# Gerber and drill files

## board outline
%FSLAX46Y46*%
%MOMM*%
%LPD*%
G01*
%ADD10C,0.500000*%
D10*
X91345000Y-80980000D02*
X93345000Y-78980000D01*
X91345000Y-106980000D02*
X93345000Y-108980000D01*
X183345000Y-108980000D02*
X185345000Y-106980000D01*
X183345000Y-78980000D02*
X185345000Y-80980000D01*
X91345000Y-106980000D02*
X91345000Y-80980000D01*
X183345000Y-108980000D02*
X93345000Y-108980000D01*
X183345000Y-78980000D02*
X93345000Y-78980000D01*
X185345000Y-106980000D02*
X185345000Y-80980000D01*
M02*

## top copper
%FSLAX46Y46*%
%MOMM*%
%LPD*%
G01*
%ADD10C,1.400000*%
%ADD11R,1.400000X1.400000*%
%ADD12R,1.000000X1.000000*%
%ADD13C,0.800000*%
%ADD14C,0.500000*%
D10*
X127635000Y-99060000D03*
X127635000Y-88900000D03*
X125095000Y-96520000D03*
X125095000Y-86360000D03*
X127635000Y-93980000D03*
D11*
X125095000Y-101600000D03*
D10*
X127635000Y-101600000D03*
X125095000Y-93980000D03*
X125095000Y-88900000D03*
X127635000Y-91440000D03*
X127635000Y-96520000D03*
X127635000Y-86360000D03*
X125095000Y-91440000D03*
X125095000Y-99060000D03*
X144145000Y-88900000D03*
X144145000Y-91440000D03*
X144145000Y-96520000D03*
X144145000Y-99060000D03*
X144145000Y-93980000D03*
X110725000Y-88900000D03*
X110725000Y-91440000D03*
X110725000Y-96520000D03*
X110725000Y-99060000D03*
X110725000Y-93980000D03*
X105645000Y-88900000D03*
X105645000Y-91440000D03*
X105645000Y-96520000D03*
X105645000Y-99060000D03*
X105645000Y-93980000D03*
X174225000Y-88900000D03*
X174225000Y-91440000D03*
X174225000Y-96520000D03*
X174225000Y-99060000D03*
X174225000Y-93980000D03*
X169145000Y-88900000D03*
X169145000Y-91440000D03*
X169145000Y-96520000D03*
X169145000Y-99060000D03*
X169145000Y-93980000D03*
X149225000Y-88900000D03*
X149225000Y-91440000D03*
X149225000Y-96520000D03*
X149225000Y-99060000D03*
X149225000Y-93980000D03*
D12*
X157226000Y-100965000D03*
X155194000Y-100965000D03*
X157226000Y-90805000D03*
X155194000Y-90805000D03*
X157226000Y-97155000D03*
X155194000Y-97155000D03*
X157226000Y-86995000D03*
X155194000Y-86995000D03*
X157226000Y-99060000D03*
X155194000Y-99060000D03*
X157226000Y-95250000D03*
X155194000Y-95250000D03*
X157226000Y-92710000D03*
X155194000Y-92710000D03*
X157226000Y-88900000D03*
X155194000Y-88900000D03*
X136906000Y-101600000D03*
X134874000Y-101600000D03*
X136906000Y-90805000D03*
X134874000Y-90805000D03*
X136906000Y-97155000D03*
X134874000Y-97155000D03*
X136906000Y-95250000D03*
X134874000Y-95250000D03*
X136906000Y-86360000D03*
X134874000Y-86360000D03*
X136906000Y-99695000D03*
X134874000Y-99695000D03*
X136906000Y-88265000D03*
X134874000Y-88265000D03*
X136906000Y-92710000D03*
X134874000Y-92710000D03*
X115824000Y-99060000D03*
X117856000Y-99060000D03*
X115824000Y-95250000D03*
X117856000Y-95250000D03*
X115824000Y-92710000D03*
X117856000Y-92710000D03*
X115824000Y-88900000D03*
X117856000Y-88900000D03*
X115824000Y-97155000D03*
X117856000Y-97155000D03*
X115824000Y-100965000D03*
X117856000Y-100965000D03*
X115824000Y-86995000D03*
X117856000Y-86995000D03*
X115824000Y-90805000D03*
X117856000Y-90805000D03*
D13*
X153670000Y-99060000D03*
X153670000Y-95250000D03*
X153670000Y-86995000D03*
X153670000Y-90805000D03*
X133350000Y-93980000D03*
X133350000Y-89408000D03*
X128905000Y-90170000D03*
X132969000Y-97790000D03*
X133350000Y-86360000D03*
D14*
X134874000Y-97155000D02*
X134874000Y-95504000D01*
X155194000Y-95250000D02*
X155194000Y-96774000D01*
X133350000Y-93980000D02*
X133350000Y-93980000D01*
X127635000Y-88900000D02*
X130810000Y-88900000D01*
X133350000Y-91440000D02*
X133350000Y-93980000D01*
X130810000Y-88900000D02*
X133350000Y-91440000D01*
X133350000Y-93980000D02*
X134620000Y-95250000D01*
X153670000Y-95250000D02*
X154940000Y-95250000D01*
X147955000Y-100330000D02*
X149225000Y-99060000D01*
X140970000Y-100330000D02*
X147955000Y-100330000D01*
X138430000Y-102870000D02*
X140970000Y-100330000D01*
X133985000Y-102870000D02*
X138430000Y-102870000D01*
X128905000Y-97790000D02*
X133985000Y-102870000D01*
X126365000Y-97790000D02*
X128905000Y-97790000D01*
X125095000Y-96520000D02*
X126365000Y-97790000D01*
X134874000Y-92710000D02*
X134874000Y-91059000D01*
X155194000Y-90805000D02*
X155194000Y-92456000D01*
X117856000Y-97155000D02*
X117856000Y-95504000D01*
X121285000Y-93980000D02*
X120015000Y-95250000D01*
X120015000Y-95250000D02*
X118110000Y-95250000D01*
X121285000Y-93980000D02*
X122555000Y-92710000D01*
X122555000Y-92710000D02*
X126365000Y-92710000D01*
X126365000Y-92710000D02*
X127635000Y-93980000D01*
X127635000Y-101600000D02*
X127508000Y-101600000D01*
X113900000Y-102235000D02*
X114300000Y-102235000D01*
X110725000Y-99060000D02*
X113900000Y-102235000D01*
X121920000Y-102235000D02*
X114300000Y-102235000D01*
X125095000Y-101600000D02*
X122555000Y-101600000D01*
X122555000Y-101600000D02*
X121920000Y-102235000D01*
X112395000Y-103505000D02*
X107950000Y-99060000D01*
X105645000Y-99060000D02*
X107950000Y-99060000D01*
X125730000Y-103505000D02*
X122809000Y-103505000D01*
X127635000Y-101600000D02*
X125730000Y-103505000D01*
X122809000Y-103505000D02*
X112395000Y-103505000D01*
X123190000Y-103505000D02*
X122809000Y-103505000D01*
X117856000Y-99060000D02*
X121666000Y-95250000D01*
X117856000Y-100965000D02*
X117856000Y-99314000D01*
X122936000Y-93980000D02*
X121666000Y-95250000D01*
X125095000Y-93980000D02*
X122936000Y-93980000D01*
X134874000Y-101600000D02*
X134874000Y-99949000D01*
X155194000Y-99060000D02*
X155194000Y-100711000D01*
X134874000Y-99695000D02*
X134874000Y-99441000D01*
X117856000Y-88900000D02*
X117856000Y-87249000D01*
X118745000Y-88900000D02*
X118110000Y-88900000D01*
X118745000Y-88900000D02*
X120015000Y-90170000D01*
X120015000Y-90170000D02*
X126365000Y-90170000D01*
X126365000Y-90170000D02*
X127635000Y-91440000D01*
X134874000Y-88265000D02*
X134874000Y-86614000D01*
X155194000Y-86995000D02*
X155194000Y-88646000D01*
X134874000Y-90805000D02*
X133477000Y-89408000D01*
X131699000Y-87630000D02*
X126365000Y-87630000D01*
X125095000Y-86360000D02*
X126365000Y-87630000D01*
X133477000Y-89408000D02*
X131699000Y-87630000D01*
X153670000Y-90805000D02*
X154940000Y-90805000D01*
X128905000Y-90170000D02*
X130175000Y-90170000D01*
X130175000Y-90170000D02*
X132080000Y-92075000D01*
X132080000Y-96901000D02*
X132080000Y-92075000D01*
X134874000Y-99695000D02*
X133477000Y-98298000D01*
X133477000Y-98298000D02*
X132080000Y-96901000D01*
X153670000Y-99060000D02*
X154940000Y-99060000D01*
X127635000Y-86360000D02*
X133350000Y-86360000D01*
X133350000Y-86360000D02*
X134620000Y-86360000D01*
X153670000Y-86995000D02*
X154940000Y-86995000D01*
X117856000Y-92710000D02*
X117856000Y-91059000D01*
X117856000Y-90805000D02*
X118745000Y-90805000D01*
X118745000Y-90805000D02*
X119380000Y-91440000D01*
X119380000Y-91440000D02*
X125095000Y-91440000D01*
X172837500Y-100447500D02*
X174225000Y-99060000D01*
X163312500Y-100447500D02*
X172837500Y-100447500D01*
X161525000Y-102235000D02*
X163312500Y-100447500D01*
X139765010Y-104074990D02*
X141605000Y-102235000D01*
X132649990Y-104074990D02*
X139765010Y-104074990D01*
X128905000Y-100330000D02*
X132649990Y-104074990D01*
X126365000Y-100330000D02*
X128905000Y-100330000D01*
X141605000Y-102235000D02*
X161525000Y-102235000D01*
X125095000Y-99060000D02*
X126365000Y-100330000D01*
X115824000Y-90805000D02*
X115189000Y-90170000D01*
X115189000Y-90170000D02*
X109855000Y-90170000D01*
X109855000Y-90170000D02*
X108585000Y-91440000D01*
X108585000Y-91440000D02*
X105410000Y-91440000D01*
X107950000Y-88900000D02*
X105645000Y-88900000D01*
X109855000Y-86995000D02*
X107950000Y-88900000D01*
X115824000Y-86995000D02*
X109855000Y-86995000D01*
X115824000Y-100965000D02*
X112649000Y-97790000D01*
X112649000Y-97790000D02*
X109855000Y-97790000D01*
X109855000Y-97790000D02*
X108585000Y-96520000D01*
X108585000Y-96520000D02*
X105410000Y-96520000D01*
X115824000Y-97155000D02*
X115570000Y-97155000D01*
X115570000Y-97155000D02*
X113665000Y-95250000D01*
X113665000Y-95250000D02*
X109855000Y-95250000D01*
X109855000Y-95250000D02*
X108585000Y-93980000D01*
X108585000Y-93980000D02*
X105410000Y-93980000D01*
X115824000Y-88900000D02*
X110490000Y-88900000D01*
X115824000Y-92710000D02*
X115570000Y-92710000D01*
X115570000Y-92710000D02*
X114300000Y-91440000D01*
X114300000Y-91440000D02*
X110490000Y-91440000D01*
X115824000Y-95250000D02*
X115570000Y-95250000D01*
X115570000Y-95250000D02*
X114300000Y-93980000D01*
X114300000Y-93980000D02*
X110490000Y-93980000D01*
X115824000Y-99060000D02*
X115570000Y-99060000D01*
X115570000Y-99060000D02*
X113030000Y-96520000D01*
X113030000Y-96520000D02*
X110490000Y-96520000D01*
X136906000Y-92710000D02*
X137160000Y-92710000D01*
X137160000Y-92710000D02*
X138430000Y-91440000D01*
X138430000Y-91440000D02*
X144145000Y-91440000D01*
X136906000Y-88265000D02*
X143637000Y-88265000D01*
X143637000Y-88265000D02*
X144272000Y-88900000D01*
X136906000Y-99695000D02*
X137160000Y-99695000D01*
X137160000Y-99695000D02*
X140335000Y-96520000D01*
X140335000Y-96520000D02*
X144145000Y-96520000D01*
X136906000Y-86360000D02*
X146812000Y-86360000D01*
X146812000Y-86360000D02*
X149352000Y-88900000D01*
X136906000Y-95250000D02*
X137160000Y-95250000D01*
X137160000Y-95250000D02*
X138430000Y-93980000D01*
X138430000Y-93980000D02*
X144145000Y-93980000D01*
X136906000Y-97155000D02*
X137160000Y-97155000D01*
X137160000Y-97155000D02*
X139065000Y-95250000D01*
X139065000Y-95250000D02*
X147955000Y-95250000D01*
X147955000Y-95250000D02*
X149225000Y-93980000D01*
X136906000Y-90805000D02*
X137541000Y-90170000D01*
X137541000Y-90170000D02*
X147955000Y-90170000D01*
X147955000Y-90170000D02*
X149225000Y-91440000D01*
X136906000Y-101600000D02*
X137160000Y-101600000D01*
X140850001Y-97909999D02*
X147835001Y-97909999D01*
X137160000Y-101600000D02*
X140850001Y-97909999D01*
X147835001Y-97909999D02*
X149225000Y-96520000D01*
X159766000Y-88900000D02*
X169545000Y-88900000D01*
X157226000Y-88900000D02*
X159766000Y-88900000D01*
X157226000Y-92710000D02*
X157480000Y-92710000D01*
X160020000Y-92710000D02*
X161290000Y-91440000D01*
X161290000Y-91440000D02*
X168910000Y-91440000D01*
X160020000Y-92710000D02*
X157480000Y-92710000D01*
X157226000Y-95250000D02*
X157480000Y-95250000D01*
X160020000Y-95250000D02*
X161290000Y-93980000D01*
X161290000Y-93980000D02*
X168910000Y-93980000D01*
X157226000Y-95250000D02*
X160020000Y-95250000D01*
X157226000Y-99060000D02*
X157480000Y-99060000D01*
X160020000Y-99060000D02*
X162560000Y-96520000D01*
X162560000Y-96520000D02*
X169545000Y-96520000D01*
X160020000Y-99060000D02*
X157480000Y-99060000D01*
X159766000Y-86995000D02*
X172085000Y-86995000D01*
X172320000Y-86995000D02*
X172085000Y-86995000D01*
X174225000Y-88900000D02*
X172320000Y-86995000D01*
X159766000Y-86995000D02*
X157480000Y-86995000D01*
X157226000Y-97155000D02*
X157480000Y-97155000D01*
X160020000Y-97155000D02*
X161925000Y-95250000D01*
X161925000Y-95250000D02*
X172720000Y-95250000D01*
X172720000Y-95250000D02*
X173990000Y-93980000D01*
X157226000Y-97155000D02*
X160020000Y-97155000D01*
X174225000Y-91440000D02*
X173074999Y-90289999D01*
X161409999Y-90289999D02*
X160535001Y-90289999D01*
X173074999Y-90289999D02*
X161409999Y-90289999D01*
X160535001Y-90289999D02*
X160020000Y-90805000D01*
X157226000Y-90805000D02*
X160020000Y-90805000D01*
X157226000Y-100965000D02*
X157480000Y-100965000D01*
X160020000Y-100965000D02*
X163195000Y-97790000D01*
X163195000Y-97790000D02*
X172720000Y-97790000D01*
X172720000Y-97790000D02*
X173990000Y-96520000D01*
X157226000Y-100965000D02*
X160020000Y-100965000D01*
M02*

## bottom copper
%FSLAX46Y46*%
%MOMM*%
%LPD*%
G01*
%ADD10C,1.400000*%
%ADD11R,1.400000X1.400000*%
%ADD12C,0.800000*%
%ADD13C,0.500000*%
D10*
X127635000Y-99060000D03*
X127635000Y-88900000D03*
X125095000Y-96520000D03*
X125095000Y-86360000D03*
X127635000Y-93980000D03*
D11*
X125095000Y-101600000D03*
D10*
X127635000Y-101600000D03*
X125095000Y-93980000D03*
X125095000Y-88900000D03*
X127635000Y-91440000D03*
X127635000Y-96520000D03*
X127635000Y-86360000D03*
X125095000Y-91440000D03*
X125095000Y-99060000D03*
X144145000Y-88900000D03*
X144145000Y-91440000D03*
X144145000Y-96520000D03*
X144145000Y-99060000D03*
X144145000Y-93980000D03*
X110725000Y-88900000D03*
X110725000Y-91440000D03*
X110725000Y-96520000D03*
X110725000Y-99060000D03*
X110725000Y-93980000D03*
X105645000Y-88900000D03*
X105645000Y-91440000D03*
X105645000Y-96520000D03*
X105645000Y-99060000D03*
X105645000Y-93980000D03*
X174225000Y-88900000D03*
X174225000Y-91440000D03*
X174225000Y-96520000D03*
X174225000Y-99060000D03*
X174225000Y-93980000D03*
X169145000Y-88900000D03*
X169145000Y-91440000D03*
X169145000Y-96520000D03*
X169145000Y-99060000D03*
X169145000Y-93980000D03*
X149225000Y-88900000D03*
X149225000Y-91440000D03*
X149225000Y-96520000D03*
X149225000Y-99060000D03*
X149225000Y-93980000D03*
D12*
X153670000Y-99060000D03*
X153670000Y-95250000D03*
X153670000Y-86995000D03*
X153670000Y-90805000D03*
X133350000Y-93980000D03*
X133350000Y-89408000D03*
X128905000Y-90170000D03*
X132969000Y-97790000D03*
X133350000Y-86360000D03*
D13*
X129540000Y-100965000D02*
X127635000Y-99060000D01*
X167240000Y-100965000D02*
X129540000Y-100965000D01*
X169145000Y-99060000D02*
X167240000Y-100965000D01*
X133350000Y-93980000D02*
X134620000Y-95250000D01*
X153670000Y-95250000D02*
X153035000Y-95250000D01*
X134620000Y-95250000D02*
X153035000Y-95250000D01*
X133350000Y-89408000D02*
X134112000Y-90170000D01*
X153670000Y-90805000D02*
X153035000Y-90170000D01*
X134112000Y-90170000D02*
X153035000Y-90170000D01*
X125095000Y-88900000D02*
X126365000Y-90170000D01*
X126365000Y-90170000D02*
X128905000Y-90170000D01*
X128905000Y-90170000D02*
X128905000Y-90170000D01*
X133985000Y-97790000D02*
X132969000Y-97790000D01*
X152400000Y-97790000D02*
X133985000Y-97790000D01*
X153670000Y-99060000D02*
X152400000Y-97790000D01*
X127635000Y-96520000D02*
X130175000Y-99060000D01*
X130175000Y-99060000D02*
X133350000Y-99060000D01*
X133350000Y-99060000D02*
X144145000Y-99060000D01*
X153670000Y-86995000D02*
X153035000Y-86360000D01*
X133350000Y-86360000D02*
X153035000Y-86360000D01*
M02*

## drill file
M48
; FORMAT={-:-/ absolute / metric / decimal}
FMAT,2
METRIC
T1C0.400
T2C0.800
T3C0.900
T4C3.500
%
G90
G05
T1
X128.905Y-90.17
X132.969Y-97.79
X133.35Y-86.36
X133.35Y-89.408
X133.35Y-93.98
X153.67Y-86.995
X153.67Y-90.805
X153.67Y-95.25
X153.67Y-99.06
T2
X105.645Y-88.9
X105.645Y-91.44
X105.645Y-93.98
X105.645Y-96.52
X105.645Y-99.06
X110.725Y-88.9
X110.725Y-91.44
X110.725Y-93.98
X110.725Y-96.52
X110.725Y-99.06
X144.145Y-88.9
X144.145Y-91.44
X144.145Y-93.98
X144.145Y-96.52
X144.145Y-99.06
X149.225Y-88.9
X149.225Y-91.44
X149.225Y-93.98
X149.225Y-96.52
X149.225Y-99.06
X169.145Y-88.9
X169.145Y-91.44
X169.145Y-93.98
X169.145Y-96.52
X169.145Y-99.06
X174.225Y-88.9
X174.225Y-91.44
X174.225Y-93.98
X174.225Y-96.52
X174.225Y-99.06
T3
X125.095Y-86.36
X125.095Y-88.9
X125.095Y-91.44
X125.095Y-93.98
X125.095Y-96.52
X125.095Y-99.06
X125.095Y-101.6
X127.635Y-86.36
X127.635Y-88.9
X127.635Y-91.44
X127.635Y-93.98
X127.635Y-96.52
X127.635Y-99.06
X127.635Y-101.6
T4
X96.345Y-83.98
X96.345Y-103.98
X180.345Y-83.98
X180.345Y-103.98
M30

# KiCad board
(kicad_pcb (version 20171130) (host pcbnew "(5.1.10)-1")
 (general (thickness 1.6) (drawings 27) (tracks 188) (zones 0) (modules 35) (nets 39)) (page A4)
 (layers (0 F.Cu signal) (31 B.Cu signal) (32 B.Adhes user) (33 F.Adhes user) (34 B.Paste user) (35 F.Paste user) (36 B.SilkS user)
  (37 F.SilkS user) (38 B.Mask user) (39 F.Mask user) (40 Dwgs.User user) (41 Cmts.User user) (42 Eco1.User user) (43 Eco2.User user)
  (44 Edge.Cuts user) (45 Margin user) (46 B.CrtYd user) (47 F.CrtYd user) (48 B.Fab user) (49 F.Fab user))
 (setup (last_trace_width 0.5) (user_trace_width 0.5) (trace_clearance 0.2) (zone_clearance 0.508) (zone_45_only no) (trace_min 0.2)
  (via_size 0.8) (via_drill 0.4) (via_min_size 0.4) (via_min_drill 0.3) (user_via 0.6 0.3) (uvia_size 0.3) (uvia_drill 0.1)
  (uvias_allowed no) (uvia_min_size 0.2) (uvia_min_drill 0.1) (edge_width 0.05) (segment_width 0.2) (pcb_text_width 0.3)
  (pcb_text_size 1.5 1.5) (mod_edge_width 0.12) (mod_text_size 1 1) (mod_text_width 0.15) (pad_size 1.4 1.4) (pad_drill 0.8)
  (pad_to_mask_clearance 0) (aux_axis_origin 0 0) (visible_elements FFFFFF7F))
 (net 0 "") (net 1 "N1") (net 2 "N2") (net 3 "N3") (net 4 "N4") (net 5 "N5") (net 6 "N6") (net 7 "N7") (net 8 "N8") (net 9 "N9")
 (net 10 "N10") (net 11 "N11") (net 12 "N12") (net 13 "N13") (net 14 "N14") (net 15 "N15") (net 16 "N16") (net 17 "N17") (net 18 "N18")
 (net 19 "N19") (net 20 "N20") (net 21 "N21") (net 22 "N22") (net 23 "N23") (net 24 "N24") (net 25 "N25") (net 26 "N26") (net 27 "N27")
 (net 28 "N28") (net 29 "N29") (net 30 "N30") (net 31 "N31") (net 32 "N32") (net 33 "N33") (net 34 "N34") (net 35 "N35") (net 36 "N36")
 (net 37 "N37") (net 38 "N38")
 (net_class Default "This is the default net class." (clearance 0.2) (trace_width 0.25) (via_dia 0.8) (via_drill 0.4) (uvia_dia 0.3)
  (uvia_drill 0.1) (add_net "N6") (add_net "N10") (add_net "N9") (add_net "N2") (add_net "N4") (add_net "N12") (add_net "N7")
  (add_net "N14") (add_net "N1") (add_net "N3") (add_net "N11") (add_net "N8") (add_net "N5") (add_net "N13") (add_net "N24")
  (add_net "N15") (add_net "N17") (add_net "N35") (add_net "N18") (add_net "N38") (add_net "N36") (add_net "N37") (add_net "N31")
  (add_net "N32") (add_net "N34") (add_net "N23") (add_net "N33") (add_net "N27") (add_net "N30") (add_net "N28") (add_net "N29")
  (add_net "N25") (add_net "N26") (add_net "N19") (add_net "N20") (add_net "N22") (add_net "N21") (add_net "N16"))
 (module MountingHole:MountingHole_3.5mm (layer F.Cu) (at 96.345 103.98)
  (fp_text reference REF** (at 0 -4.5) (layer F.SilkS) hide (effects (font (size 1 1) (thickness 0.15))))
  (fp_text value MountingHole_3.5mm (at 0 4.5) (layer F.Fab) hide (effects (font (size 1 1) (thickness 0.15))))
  (pad 1 np_thru_hole circle (at 0 0) (size 3.5 3.5) (drill 3.5) (layers *.Cu *.Mask)))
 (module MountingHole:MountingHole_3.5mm (layer F.Cu) (at 96.345 83.98)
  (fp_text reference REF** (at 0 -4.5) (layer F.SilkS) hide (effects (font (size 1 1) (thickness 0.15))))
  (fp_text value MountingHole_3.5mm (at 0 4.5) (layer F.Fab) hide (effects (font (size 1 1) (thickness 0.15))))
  (pad 1 np_thru_hole circle (at 0 0) (size 3.5 3.5) (drill 3.5) (layers *.Cu *.Mask)))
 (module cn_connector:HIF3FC (layer B.Cu) (at 126.365 93.98)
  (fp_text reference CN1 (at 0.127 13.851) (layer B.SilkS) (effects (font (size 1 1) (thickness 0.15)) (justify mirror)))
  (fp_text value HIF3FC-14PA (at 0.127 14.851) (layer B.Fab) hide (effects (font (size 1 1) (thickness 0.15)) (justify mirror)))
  (pad 4 thru_hole circle (at 1.27 5.08) (size 1.4 1.4) (drill 0.9) (layers *.Cu *.Mask) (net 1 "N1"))
  (pad 12 thru_hole circle (at 1.27 -5.08) (size 1.4 1.4) (drill 0.9) (layers *.Cu *.Mask) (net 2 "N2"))
  (pad 5 thru_hole circle (at -1.27 2.54) (size 1.4 1.4) (drill 0.9) (layers *.Cu *.Mask) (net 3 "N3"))
  (pad 13 thru_hole circle (at -1.27 -7.62) (size 1.4 1.4) (drill 0.9) (layers *.Cu *.Mask) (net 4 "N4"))
  (pad 8 thru_hole circle (at 1.27 0) (size 1.4 1.4) (drill 0.9) (layers *.Cu *.Mask) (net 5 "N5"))
  (pad 1 thru_hole rect (at -1.27 7.62) (size 1.4 1.4) (drill 0.9) (layers *.Cu *.Mask) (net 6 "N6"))
  (pad 2 thru_hole circle (at 1.27 7.62) (size 1.4 1.4) (drill 0.9) (layers *.Cu *.Mask) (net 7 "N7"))
  (pad 7 thru_hole circle (at -1.27 0) (size 1.4 1.4) (drill 0.9) (layers *.Cu *.Mask) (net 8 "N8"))
  (pad 11 thru_hole circle (at -1.27 -5.08) (size 1.4 1.4) (drill 0.9) (layers *.Cu *.Mask) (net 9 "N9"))
  (pad 10 thru_hole circle (at 1.27 -2.54) (size 1.4 1.4) (drill 0.9) (layers *.Cu *.Mask) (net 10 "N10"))
  (pad 6 thru_hole circle (at 1.27 2.54) (size 1.4 1.4) (drill 0.9) (layers *.Cu *.Mask) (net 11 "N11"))
  (pad 14 thru_hole circle (at 1.27 -7.62) (size 1.4 1.4) (drill 0.9) (layers *.Cu *.Mask) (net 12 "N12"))
  (pad 9 thru_hole circle (at -1.27 -2.54) (size 1.4 1.4) (drill 0.9) (layers *.Cu *.Mask) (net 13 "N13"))
  (pad 3 thru_hole circle (at -1.27 5.08) (size 1.4 1.4) (drill 0.9) (layers *.Cu *.Mask) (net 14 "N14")))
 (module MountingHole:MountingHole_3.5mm (layer F.Cu) (at 180.345 103.98)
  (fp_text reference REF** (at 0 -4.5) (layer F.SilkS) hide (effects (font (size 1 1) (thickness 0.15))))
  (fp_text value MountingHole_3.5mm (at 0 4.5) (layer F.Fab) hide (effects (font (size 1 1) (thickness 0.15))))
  (pad 1 np_thru_hole circle (at 0 0) (size 3.5 3.5) (drill 3.5) (layers *.Cu *.Mask)))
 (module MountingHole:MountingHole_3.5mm (layer F.Cu) (at 180.345 83.98)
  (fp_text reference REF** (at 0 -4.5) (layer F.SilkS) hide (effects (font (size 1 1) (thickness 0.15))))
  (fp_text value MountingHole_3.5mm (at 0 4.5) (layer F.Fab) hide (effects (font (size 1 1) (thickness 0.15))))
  (pad 1 np_thru_hole circle (at 0 0) (size 3.5 3.5) (drill 3.5) (layers *.Cu *.Mask)))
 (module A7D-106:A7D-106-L (layer F.Cu) (at 144.145 88.9)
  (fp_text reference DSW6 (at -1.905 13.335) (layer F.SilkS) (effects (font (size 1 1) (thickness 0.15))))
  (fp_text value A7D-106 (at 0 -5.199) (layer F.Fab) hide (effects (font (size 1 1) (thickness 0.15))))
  (pad 8 thru_hole circle (at 0 0) (size 1.4 1.4) (drill 0.8) (layers *.Cu *.Mask) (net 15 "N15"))
  (pad 4 thru_hole circle (at 0 2.54) (size 1.4 1.4) (drill 0.8) (layers *.Cu *.Mask) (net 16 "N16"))
  (pad 1 thru_hole circle (at 0 7.62) (size 1.4 1.4) (drill 0.8) (layers *.Cu *.Mask) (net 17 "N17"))
  (pad C thru_hole circle (at 0 10.16) (size 1.4 1.4) (drill 0.8) (layers *.Cu *.Mask) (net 11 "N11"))
  (pad 2 thru_hole circle (at 0 5.08) (size 1.4 1.4) (drill 0.8) (layers *.Cu *.Mask) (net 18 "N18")))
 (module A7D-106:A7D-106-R (layer F.Cu) (at 110.725 88.9)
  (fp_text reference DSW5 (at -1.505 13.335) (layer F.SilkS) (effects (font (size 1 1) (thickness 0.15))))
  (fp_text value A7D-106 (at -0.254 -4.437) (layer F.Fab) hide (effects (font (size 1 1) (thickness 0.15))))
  (pad 8 thru_hole circle (at 0 0) (size 1.4 1.4) (drill 0.8) (layers *.Cu *.Mask) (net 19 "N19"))
  (pad 4 thru_hole circle (at 0 2.54) (size 1.4 1.4) (drill 0.8) (layers *.Cu *.Mask) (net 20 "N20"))
  (pad 1 thru_hole circle (at 0 7.62) (size 1.4 1.4) (drill 0.8) (layers *.Cu *.Mask) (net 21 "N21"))
  (pad C thru_hole circle (at 0 10.16) (size 1.4 1.4) (drill 0.8) (layers *.Cu *.Mask) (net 6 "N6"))
  (pad 2 thru_hole circle (at 0 5.08) (size 1.4 1.4) (drill 0.8) (layers *.Cu *.Mask) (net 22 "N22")))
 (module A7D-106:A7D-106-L (layer F.Cu) (at 105.645 88.9)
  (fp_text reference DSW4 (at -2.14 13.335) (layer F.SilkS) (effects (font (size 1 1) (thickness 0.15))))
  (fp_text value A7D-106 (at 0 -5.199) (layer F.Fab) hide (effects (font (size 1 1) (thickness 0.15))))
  (pad 8 thru_hole circle (at 0 0) (size 1.4 1.4) (drill 0.8) (layers *.Cu *.Mask) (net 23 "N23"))
  (pad 4 thru_hole circle (at 0 2.54) (size 1.4 1.4) (drill 0.8) (layers *.Cu *.Mask) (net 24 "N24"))
  (pad 1 thru_hole circle (at 0 7.62) (size 1.4 1.4) (drill 0.8) (layers *.Cu *.Mask) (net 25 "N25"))
  (pad C thru_hole circle (at 0 10.16) (size 1.4 1.4) (drill 0.8) (layers *.Cu *.Mask) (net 7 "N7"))
  (pad 2 thru_hole circle (at 0 5.08) (size 1.4 1.4) (drill 0.8) (layers *.Cu *.Mask) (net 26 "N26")))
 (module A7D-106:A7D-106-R (layer F.Cu) (at 174.225 88.9)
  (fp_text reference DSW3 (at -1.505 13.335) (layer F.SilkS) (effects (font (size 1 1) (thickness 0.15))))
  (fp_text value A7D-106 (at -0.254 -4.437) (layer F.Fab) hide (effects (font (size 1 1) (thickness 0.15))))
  (pad 8 thru_hole circle (at 0 0) (size 1.4 1.4) (drill 0.8) (layers *.Cu *.Mask) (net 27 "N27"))
  (pad 4 thru_hole circle (at 0 2.54) (size 1.4 1.4) (drill 0.8) (layers *.Cu *.Mask) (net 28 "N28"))
  (pad 1 thru_hole circle (at 0 7.62) (size 1.4 1.4) (drill 0.8) (layers *.Cu *.Mask) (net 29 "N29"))
  (pad C thru_hole circle (at 0 10.16) (size 1.4 1.4) (drill 0.8) (layers *.Cu *.Mask) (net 14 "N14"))
  (pad 2 thru_hole circle (at 0 5.08) (size 1.4 1.4) (drill 0.8) (layers *.Cu *.Mask) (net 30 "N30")))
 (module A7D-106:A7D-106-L (layer F.Cu) (at 169.145 88.9)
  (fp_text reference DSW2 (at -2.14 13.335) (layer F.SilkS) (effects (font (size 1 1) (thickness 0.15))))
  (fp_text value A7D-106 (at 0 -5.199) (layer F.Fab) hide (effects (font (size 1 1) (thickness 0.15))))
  (pad 8 thru_hole circle (at 0 0) (size 1.4 1.4) (drill 0.8) (layers *.Cu *.Mask) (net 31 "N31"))
  (pad 4 thru_hole circle (at 0 2.54) (size 1.4 1.4) (drill 0.8) (layers *.Cu *.Mask) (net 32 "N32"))
  (pad 1 thru_hole circle (at 0 7.62) (size 1.4 1.4) (drill 0.8) (layers *.Cu *.Mask) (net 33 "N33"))
  (pad C thru_hole circle (at 0 10.16) (size 1.4 1.4) (drill 0.8) (layers *.Cu *.Mask) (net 1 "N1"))
  (pad 2 thru_hole circle (at 0 5.08) (size 1.4 1.4) (drill 0.8) (layers *.Cu *.Mask) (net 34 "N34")))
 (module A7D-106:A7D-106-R (layer F.Cu) (at 149.225 88.9)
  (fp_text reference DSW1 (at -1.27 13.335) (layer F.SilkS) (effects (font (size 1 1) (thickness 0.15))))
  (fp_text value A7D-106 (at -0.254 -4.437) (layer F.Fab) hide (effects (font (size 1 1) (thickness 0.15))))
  (pad 8 thru_hole circle (at 0 0) (size 1.4 1.4) (drill 0.8) (layers *.Cu *.Mask) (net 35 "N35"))
  (pad 4 thru_hole circle (at 0 2.54) (size 1.4 1.4) (drill 0.8) (layers *.Cu *.Mask) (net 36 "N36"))
  (pad 1 thru_hole circle (at 0 7.62) (size 1.4 1.4) (drill 0.8) (layers *.Cu *.Mask) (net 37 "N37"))
  (pad C thru_hole circle (at 0 10.16) (size 1.4 1.4) (drill 0.8) (layers *.Cu *.Mask) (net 3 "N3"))
  (pad 2 thru_hole circle (at 0 5.08) (size 1.4 1.4) (drill 0.8) (layers *.Cu *.Mask) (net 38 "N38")))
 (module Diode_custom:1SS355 (layer F.Cu) (at 156.21 100.965)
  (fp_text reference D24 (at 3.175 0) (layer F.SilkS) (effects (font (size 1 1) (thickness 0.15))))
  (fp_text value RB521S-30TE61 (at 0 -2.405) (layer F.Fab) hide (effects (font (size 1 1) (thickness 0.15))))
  (pad 2 smd rect (at 1.016 0) (size 1 1) (layers F.Cu F.Paste F.Mask) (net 29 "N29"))
  (pad 1 smd rect (at -1.016 0) (size 1 1) (layers F.Cu F.Paste F.Mask) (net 9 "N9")))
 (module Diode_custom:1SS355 (layer F.Cu) (at 156.21 90.805)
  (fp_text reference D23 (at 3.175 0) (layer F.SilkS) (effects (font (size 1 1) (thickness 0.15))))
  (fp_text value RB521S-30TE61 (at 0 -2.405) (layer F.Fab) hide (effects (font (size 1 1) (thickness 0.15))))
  (pad 2 smd rect (at 1.016 0) (size 1 1) (layers F.Cu F.Paste F.Mask) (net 28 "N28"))
  (pad 1 smd rect (at -1.016 0) (size 1 1) (layers F.Cu F.Paste F.Mask) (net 4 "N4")))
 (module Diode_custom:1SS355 (layer F.Cu) (at 156.21 97.155)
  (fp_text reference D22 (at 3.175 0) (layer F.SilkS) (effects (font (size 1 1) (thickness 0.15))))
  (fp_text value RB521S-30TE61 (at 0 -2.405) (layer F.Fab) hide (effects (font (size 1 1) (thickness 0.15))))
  (pad 2 smd rect (at 1.016 0) (size 1 1) (layers F.Cu F.Paste F.Mask) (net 30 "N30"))
  (pad 1 smd rect (at -1.016 0) (size 1 1) (layers F.Cu F.Paste F.Mask) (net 2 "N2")))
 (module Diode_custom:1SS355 (layer F.Cu) (at 156.21 86.995)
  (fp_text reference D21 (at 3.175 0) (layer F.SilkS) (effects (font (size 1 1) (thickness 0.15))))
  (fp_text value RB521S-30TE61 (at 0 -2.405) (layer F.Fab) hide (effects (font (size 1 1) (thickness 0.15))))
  (pad 2 smd rect (at 1.016 0) (size 1 1) (layers F.Cu F.Paste F.Mask) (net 27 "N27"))
  (pad 1 smd rect (at -1.016 0) (size 1 1) (layers F.Cu F.Paste F.Mask) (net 12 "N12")))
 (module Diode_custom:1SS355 (layer F.Cu) (at 156.21 99.06)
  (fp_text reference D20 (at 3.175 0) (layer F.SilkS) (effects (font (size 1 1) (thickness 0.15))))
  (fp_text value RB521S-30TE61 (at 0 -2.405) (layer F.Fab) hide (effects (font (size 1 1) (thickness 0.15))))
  (pad 2 smd rect (at 1.016 0) (size 1 1) (layers F.Cu F.Paste F.Mask) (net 33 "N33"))
  (pad 1 smd rect (at -1.016 0) (size 1 1) (layers F.Cu F.Paste F.Mask) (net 9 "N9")))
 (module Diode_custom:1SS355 (layer F.Cu) (at 156.21 95.25)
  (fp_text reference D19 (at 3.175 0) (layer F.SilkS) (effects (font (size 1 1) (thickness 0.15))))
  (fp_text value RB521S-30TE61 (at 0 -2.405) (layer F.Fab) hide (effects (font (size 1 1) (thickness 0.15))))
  (pad 2 smd rect (at 1.016 0) (size 1 1) (layers F.Cu F.Paste F.Mask) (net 34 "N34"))
  (pad 1 smd rect (at -1.016 0) (size 1 1) (layers F.Cu F.Paste F.Mask) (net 2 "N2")))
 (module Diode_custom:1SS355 (layer F.Cu) (at 156.21 92.71)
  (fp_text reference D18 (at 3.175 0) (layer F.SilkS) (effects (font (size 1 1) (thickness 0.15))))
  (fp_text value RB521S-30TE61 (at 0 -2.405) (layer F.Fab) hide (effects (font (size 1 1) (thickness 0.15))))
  (pad 2 smd rect (at 1.016 0) (size 1 1) (layers F.Cu F.Paste F.Mask) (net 32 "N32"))
  (pad 1 smd rect (at -1.016 0) (size 1 1) (layers F.Cu F.Paste F.Mask) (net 4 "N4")))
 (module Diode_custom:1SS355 (layer F.Cu) (at 156.21 88.9)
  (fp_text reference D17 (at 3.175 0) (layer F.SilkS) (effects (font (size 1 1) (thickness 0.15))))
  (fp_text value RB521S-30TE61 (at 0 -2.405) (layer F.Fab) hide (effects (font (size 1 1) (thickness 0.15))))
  (pad 2 smd rect (at 1.016 0) (size 1 1) (layers F.Cu F.Paste F.Mask) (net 31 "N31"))
  (pad 1 smd rect (at -1.016 0) (size 1 1) (layers F.Cu F.Paste F.Mask) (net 12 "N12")))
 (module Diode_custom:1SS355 (layer F.Cu) (at 135.89 101.6)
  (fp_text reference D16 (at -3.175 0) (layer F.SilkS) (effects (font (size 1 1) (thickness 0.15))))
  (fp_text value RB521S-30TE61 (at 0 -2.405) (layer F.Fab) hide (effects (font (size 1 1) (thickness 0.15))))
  (pad 2 smd rect (at 1.016 0) (size 1 1) (layers F.Cu F.Paste F.Mask) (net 37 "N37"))
  (pad 1 smd rect (at -1.016 0) (size 1 1) (layers F.Cu F.Paste F.Mask) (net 9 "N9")))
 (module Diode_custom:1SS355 (layer F.Cu) (at 135.89 90.805)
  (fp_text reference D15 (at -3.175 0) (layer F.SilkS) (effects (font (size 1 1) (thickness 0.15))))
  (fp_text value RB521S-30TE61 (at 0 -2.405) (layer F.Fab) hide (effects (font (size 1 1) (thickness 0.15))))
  (pad 2 smd rect (at 1.016 0) (size 1 1) (layers F.Cu F.Paste F.Mask) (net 36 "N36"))
  (pad 1 smd rect (at -1.016 0) (size 1 1) (layers F.Cu F.Paste F.Mask) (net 4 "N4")))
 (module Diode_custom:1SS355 (layer F.Cu) (at 135.89 97.155)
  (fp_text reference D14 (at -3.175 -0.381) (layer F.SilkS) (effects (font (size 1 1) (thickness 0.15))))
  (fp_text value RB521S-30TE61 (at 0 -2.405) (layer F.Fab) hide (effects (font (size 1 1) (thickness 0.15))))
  (pad 2 smd rect (at 1.016 0) (size 1 1) (layers F.Cu F.Paste F.Mask) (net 38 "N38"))
  (pad 1 smd rect (at -1.016 0) (size 1 1) (layers F.Cu F.Paste F.Mask) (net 2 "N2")))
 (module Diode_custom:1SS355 (layer F.Cu) (at 135.89 95.25)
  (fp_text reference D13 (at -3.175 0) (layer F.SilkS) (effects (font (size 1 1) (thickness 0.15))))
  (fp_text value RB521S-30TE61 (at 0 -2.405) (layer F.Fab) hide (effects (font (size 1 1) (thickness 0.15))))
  (pad 2 smd rect (at 1.016 0) (size 1 1) (layers F.Cu F.Paste F.Mask) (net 18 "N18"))
  (pad 1 smd rect (at -1.016 0) (size 1 1) (layers F.Cu F.Paste F.Mask) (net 2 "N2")))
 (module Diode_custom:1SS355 (layer F.Cu) (at 135.89 86.36)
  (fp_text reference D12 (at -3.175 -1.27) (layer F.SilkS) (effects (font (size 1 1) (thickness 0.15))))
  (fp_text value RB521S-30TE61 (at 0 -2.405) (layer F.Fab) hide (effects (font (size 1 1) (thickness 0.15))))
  (pad 2 smd rect (at 1.016 0) (size 1 1) (layers F.Cu F.Paste F.Mask) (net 35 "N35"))
  (pad 1 smd rect (at -1.016 0) (size 1 1) (layers F.Cu F.Paste F.Mask) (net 12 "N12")))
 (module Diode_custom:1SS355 (layer F.Cu) (at 135.89 99.695)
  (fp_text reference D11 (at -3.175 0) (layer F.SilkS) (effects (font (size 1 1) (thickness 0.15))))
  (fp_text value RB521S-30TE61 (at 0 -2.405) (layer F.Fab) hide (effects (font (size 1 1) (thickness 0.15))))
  (pad 2 smd rect (at 1.016 0) (size 1 1) (layers F.Cu F.Paste F.Mask) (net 17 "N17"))
  (pad 1 smd rect (at -1.016 0) (size 1 1) (layers F.Cu F.Paste F.Mask) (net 9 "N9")))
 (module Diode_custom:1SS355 (layer F.Cu) (at 135.89 88.265)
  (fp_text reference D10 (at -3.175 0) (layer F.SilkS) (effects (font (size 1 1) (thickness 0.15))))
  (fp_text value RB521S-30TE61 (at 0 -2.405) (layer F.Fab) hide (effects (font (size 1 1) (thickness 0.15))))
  (pad 2 smd rect (at 1.016 0) (size 1 1) (layers F.Cu F.Paste F.Mask) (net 15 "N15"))
  (pad 1 smd rect (at -1.016 0) (size 1 1) (layers F.Cu F.Paste F.Mask) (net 12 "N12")))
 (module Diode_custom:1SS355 (layer F.Cu) (at 135.89 92.71)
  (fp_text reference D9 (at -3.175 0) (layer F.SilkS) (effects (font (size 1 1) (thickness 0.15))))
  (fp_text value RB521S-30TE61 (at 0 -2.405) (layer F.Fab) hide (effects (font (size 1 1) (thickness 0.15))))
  (pad 2 smd rect (at 1.016 0) (size 1 1) (layers F.Cu F.Paste F.Mask) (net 16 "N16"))
  (pad 1 smd rect (at -1.016 0) (size 1 1) (layers F.Cu F.Paste F.Mask) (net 4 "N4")))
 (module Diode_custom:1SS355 (layer F.Cu) (at 116.84 99.06 180)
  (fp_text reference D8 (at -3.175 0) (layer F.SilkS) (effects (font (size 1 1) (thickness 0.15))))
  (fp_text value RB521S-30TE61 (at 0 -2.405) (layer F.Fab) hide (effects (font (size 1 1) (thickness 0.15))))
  (pad 2 smd rect (at 1.016 0 180) (size 1 1) (layers F.Cu F.Paste F.Mask) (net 21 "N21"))
  (pad 1 smd rect (at -1.016 0 180) (size 1 1) (layers F.Cu F.Paste F.Mask) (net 8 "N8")))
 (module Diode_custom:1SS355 (layer F.Cu) (at 116.84 95.25 180)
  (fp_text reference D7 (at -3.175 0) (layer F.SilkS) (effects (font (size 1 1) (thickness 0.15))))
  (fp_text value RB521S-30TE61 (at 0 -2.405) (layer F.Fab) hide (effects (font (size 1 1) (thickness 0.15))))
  (pad 2 smd rect (at 1.016 0 180) (size 1 1) (layers F.Cu F.Paste F.Mask) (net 22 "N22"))
  (pad 1 smd rect (at -1.016 0 180) (size 1 1) (layers F.Cu F.Paste F.Mask) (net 5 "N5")))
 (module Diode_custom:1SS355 (layer F.Cu) (at 116.84 92.71 180)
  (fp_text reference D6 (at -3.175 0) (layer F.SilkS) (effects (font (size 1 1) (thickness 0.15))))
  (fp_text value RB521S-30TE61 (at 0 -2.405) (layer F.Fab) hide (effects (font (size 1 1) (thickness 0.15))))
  (pad 2 smd rect (at 1.016 0 180) (size 1 1) (layers F.Cu F.Paste F.Mask) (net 20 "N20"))
  (pad 1 smd rect (at -1.016 0 180) (size 1 1) (layers F.Cu F.Paste F.Mask) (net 13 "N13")))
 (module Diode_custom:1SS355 (layer F.Cu) (at 116.84 88.9 180)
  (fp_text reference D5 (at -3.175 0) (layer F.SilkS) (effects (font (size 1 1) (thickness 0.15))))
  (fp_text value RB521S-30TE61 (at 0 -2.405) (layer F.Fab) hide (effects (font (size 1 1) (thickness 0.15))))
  (pad 2 smd rect (at 1.016 0 180) (size 1 1) (layers F.Cu F.Paste F.Mask) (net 19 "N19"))
  (pad 1 smd rect (at -1.016 0 180) (size 1 1) (layers F.Cu F.Paste F.Mask) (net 10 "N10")))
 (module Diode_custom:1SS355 (layer F.Cu) (at 116.84 97.155 180)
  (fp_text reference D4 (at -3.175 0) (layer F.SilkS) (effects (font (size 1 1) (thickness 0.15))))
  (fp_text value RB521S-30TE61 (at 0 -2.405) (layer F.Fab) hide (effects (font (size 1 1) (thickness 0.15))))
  (pad 2 smd rect (at 1.016 0 180) (size 1 1) (layers F.Cu F.Paste F.Mask) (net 26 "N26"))
  (pad 1 smd rect (at -1.016 0 180) (size 1 1) (layers F.Cu F.Paste F.Mask) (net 5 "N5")))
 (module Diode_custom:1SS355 (layer F.Cu) (at 116.84 100.965 180)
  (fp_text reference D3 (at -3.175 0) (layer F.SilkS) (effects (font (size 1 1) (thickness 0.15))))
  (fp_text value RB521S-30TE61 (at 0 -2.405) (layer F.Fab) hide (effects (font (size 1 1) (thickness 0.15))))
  (pad 2 smd rect (at 1.016 0 180) (size 1 1) (layers F.Cu F.Paste F.Mask) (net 25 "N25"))
  (pad 1 smd rect (at -1.016 0 180) (size 1 1) (layers F.Cu F.Paste F.Mask) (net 8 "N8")))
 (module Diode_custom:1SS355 (layer F.Cu) (at 116.84 86.995 180)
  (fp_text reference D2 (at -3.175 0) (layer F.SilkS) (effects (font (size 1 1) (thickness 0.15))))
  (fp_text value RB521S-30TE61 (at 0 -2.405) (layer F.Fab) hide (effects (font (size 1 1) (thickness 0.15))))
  (pad 2 smd rect (at 1.016 0 180) (size 1 1) (layers F.Cu F.Paste F.Mask) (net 23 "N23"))
  (pad 1 smd rect (at -1.016 0 180) (size 1 1) (layers F.Cu F.Paste F.Mask) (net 10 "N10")))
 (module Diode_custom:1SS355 (layer F.Cu) (at 116.84 90.805 180)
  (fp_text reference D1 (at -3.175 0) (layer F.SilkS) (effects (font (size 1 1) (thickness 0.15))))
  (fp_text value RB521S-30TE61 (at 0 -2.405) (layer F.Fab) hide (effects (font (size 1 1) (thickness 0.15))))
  (pad 2 smd rect (at 1.016 0 180) (size 1 1) (layers F.Cu F.Paste F.Mask) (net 24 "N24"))
  (pad 1 smd rect (at -1.016 0 180) (size 1 1) (layers F.Cu F.Paste F.Mask) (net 13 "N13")))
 (gr_line (start 91.345 80.98) (end 93.345 78.98) (layer Edge.Cuts) (width 0.5))
 (gr_line (start 91.345 106.98) (end 93.345 108.98) (layer Edge.Cuts) (width 0.5))
 (gr_line (start 183.345 108.98) (end 185.345 106.98) (layer Edge.Cuts) (width 0.5))
 (gr_line (start 183.345 78.98) (end 185.345 80.98) (layer Edge.Cuts) (width 0.5))
 (gr_line (start 91.345 106.98) (end 91.345 80.98) (layer Edge.Cuts) (width 0.5))
 (gr_line (start 183.345 108.98) (end 93.345 108.98) (layer Edge.Cuts) (width 0.5))
 (gr_line (start 183.345 78.98) (end 93.345 78.98) (layer Edge.Cuts) (width 0.5))
 (gr_line (start 185.345 106.98) (end 185.345 80.98) (layer Edge.Cuts) (width 0.5))
 (segment (start 129.54 100.965) (end 127.635 99.06) (width 0.5) (layer B.Cu) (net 1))
 (segment (start 167.24 100.965) (end 129.54 100.965) (width 0.5) (layer B.Cu) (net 1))
 (segment (start 169.145 99.06) (end 167.24 100.965) (width 0.5) (layer B.Cu) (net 1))
 (via (at 153.67 99.06) (size 0.8) (drill 0.4) (layers F.Cu B.Cu) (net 9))
 (via (at 153.67 95.25) (size 0.8) (drill 0.4) (layers F.Cu B.Cu) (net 2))
 (via (at 153.67 86.995) (size 0.8) (drill 0.4) (layers F.Cu B.Cu) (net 12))
 (via (at 153.67 90.805) (size 0.8) (drill 0.4) (layers F.Cu B.Cu) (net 4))
 (segment (start 134.874 97.155) (end 134.874 95.504) (width 0.5) (layer F.Cu) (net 2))
 (segment (start 155.194 95.25) (end 155.194 96.774) (width 0.5) (layer F.Cu) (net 2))
 (segment (start 133.35 93.98) (end 133.35 93.98) (width 0.5) (layer F.Cu) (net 2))
 (segment (start 127.635 88.9) (end 130.81 88.9) (width 0.5) (layer F.Cu) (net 2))
 (segment (start 133.35 91.44) (end 133.35 93.98) (width 0.5) (layer F.Cu) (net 2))
 (segment (start 130.81 88.9) (end 133.35 91.44) (width 0.5) (layer F.Cu) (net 2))
 (segment (start 133.35 93.98) (end 134.62 95.25) (width 0.5) (layer F.Cu) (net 2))
 (via (at 133.35 93.98) (size 0.8) (drill 0.4) (layers F.Cu B.Cu) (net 2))
 (segment (start 133.35 93.98) (end 134.62 95.25) (width 0.5) (layer B.Cu) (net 2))
 (segment (start 153.67 95.25) (end 153.035 95.25) (width 0.5) (layer B.Cu) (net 2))
 (segment (start 134.62 95.25) (end 153.035 95.25) (width 0.5) (layer B.Cu) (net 2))
 (segment (start 153.67 95.25) (end 154.94 95.25) (width 0.5) (layer F.Cu) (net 2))
 (segment (start 147.955 100.33) (end 149.225 99.06) (width 0.5) (layer F.Cu) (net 3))
 (segment (start 140.97 100.33) (end 147.955 100.33) (width 0.5) (layer F.Cu) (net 3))
 (segment (start 138.43 102.87) (end 140.97 100.33) (width 0.5) (layer F.Cu) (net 3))
 (segment (start 133.985 102.87) (end 138.43 102.87) (width 0.5) (layer F.Cu) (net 3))
 (segment (start 128.905 97.79) (end 133.985 102.87) (width 0.5) (layer F.Cu) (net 3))
 (segment (start 126.365 97.79) (end 128.905 97.79) (width 0.5) (layer F.Cu) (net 3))
 (segment (start 125.095 96.52) (end 126.365 97.79) (width 0.5) (layer F.Cu) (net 3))
 (segment (start 134.874 92.71) (end 134.874 91.059) (width 0.5) (layer F.Cu) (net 4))
 (segment (start 155.194 90.805) (end 155.194 92.456) (width 0.5) (layer F.Cu) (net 4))
 (segment (start 117.856 97.155) (end 117.856 95.504) (width 0.5) (layer F.Cu) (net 5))
 (segment (start 121.285 93.98) (end 120.015 95.25) (width 0.5) (layer F.Cu) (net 5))
 (segment (start 120.015 95.25) (end 118.11 95.25) (width 0.5) (layer F.Cu) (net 5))
 (segment (start 121.285 93.98) (end 122.555 92.71) (width 0.5) (layer F.Cu) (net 5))
 (segment (start 122.555 92.71) (end 126.365 92.71) (width 0.5) (layer F.Cu) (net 5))
 (segment (start 126.365 92.71) (end 127.635 93.98) (width 0.5) (layer F.Cu) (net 5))
 (segment (start 127.635 101.6) (end 127.508 101.6) (width 0.5) (layer F.Cu) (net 7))
 (segment (start 113.9 102.235) (end 114.3 102.235) (width 0.5) (layer F.Cu) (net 6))
 (segment (start 110.725 99.06) (end 113.9 102.235) (width 0.5) (layer F.Cu) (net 6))
 (segment (start 121.92 102.235) (end 114.3 102.235) (width 0.5) (layer F.Cu) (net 6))
 (segment (start 125.095 101.6) (end 122.555 101.6) (width 0.5) (layer F.Cu) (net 6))
 (segment (start 122.555 101.6) (end 121.92 102.235) (width 0.5) (layer F.Cu) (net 6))
 (segment (start 112.395 103.505) (end 107.95 99.06) (width 0.5) (layer F.Cu) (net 7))
 (segment (start 105.645 99.06) (end 107.95 99.06) (width 0.5) (layer F.Cu) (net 7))
 (segment (start 125.73 103.505) (end 122.809 103.505) (width 0.5) (layer F.Cu) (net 7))
 (segment (start 127.635 101.6) (end 125.73 103.505) (width 0.5) (layer F.Cu) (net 7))
 (segment (start 122.809 103.505) (end 112.395 103.505) (width 0.5) (layer F.Cu) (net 7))
 (segment (start 123.19 103.505) (end 122.809 103.505) (width 0.5) (layer F.Cu) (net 7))
 (segment (start 117.856 99.06) (end 121.666 95.25) (width 0.5) (layer F.Cu) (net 8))
 (segment (start 117.856 100.965) (end 117.856 99.314) (width 0.5) (layer F.Cu) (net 8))
 (segment (start 122.936 93.98) (end 121.666 95.25) (width 0.5) (layer F.Cu) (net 8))
 (segment (start 125.095 93.98) (end 122.936 93.98) (width 0.5) (layer F.Cu) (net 8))
 (segment (start 134.874 101.6) (end 134.874 99.949) (width 0.5) (layer F.Cu) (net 9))
 (segment (start 155.194 99.06) (end 155.194 100.711) (width 0.5) (layer F.Cu) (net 9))
 (segment (start 134.874 99.695) (end 134.874 99.441) (width 0.5) (layer F.Cu) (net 9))
 (segment (start 117.856 88.9) (end 117.856 87.249) (width 0.5) (layer F.Cu) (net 10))
 (segment (start 118.745 88.9) (end 118.11 88.9) (width 0.5) (layer F.Cu) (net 10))
 (segment (start 118.745 88.9) (end 120.015 90.17) (width 0.5) (layer F.Cu) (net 10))
 (segment (start 120.015 90.17) (end 126.365 90.17) (width 0.5) (layer F.Cu) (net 10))
 (segment (start 126.365 90.17) (end 127.635 91.44) (width 0.5) (layer F.Cu) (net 10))
 (segment (start 134.874 88.265) (end 134.874 86.614) (width 0.5) (layer F.Cu) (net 12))
 (segment (start 155.194 86.995) (end 155.194 88.646) (width 0.5) (layer F.Cu) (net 12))
 (segment (start 134.874 90.805) (end 133.477 89.408) (width 0.5) (layer F.Cu) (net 4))
 (segment (start 131.699 87.63) (end 126.365 87.63) (width 0.5) (layer F.Cu) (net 4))
 (segment (start 125.095 86.36) (end 126.365 87.63) (width 0.5) (layer F.Cu) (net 4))
 (segment (start 133.477 89.408) (end 131.699 87.63) (width 0.5) (layer F.Cu) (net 4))
 (via (at 133.35 89.408) (size 0.8) (drill 0.4) (layers F.Cu B.Cu) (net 4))
 (segment (start 133.35 89.408) (end 134.112 90.17) (width 0.5) (layer B.Cu) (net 4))
 (segment (start 153.67 90.805) (end 153.035 90.17) (width 0.5) (layer B.Cu) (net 4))
 (segment (start 134.112 90.17) (end 153.035 90.17) (width 0.5) (layer B.Cu) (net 4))
 (segment (start 153.67 90.805) (end 154.94 90.805) (width 0.5) (layer F.Cu) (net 4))
 (segment (start 125.095 88.9) (end 126.365 90.17) (width 0.5) (layer B.Cu) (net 9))
 (segment (start 126.365 90.17) (end 128.905 90.17) (width 0.5) (layer B.Cu) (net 9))
 (segment (start 128.905 90.17) (end 128.905 90.17) (width 0.5) (layer B.Cu) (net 9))
 (via (at 128.905 90.17) (size 0.8) (drill 0.4) (layers F.Cu B.Cu) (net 9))
 (segment (start 128.905 90.17) (end 130.175 90.17) (width 0.5) (layer F.Cu) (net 9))
 (segment (start 130.175 90.17) (end 132.08 92.075) (width 0.5) (layer F.Cu) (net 9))
 (segment (start 132.08 96.901) (end 132.08 92.075) (width 0.5) (layer F.Cu) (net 9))
 (segment (start 134.874 99.695) (end 133.477 98.298) (width 0.5) (layer F.Cu) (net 9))
 (segment (start 133.477 98.298) (end 132.08 96.901) (width 0.5) (layer F.Cu) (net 9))
 (via (at 132.969 97.79) (size 0.8) (drill 0.4) (layers F.Cu B.Cu) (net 9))
 (segment (start 153.67 99.06) (end 154.94 99.06) (width 0.5) (layer F.Cu) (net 9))
 (segment (start 133.985 97.79) (end 132.969 97.79) (width 0.5) (layer B.Cu) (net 9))
 (segment (start 152.4 97.79) (end 133.985 97.79) (width 0.5) (layer B.Cu) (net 9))
 (segment (start 153.67 99.06) (end 152.4 97.79) (width 0.5) (layer B.Cu) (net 9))
 (segment (start 127.635 96.52) (end 130.175 99.06) (width 0.5) (layer B.Cu) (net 11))
 (segment (start 130.175 99.06) (end 133.35 99.06) (width 0.5) (layer B.Cu) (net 11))
 (segment (start 133.35 99.06) (end 144.145 99.06) (width 0.5) (layer B.Cu) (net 11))
 (segment (start 127.635 86.36) (end 133.35 86.36) (width 0.5) (layer F.Cu) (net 12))
 (segment (start 133.35 86.36) (end 134.62 86.36) (width 0.5) (layer F.Cu) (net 12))
 (via (at 133.35 86.36) (size 0.8) (drill 0.4) (layers F.Cu B.Cu) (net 12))
 (segment (start 153.67 86.995) (end 153.035 86.36) (width 0.5) (layer B.Cu) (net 12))
 (segment (start 133.35 86.36) (end 153.035 86.36) (width 0.5) (layer B.Cu) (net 12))
 (segment (start 153.67 86.995) (end 154.94 86.995) (width 0.5) (layer F.Cu) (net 12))
 (segment (start 117.856 92.71) (end 117.856 91.059) (width 0.5) (layer F.Cu) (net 13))
 (segment (start 117.856 90.805) (end 118.745 90.805) (width 0.5) (layer F.Cu) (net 13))
 (segment (start 118.745 90.805) (end 119.38 91.44) (width 0.5) (layer F.Cu) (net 13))
 (segment (start 119.38 91.44) (end 125.095 91.44) (width 0.5) (layer F.Cu) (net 13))
 (segment (start 172.8375 100.4475) (end 174.225 99.06) (width 0.5) (layer F.Cu) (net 14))
 (segment (start 163.3125 100.4475) (end 172.8375 100.4475) (width 0.5) (layer F.Cu) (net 14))
 (segment (start 161.525 102.235) (end 163.3125 100.4475) (width 0.5) (layer F.Cu) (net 14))
 (segment (start 139.76501 104.07499) (end 141.605 102.235) (width 0.5) (layer F.Cu) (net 14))
 (segment (start 132.64999 104.07499) (end 139.76501 104.07499) (width 0.5) (layer F.Cu) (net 14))
 (segment (start 128.905 100.33) (end 132.64999 104.07499) (width 0.5) (layer F.Cu) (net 14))
 (segment (start 126.365 100.33) (end 128.905 100.33) (width 0.5) (layer F.Cu) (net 14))
 (segment (start 141.605 102.235) (end 161.525 102.235) (width 0.5) (layer F.Cu) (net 14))
 (segment (start 125.095 99.06) (end 126.365 100.33) (width 0.5) (layer F.Cu) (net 14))
 (segment (start 115.824 90.805) (end 115.189 90.17) (width 0.5) (layer F.Cu) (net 24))
 (segment (start 115.189 90.17) (end 109.855 90.17) (width 0.5) (layer F.Cu) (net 24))
 (segment (start 109.855 90.17) (end 108.585 91.44) (width 0.5) (layer F.Cu) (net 24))
 (segment (start 108.585 91.44) (end 105.41 91.44) (width 0.5) (layer F.Cu) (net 24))
 (segment (start 107.95 88.9) (end 105.645 88.9) (width 0.5) (layer F.Cu) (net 23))
 (segment (start 109.855 86.995) (end 107.95 88.9) (width 0.5) (layer F.Cu) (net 23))
 (segment (start 115.824 86.995) (end 109.855 86.995) (width 0.5) (layer F.Cu) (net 23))
 (segment (start 115.824 100.965) (end 112.649 97.79) (width 0.5) (layer F.Cu) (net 25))
 (segment (start 112.649 97.79) (end 109.855 97.79) (width 0.5) (layer F.Cu) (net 25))
 (segment (start 109.855 97.79) (end 108.585 96.52) (width 0.5) (layer F.Cu) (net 25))
 (segment (start 108.585 96.52) (end 105.41 96.52) (width 0.5) (layer F.Cu) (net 25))
 (segment (start 115.824 97.155) (end 115.57 97.155) (width 0.5) (layer F.Cu) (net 26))
 (segment (start 115.57 97.155) (end 113.665 95.25) (width 0.5) (layer F.Cu) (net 26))
 (segment (start 113.665 95.25) (end 109.855 95.25) (width 0.5) (layer F.Cu) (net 26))
 (segment (start 109.855 95.25) (end 108.585 93.98) (width 0.5) (layer F.Cu) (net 26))
 (segment (start 108.585 93.98) (end 105.41 93.98) (width 0.5) (layer F.Cu) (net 26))
 (segment (start 115.824 88.9) (end 110.49 88.9) (width 0.5) (layer F.Cu) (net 19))
 (segment (start 115.824 92.71) (end 115.57 92.71) (width 0.5) (layer F.Cu) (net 20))
 (segment (start 115.57 92.71) (end 114.3 91.44) (width 0.5) (layer F.Cu) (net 20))
 (segment (start 114.3 91.44) (end 110.49 91.44) (width 0.5) (layer F.Cu) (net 20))
 (segment (start 115.824 95.25) (end 115.57 95.25) (width 0.5) (layer F.Cu) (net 22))
 (segment (start 115.57 95.25) (end 114.3 93.98) (width 0.5) (layer F.Cu) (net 22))
 (segment (start 114.3 93.98) (end 110.49 93.98) (width 0.5) (layer F.Cu) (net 22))
 (segment (start 115.824 99.06) (end 115.57 99.06) (width 0.5) (layer F.Cu) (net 21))
 (segment (start 115.57 99.06) (end 113.03 96.52) (width 0.5) (layer F.Cu) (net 21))
 (segment (start 113.03 96.52) (end 110.49 96.52) (width 0.5) (layer F.Cu) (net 21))
 (segment (start 136.906 92.71) (end 137.16 92.71) (width 0.5) (layer F.Cu) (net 16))
 (segment (start 137.16 92.71) (end 138.43 91.44) (width 0.5) (layer F.Cu) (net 16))
 (segment (start 138.43 91.44) (end 144.145 91.44) (width 0.5) (layer F.Cu) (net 16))
 (segment (start 136.906 88.265) (end 143.637 88.265) (width 0.5) (layer F.Cu) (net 15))
 (segment (start 143.637 88.265) (end 144.272 88.9) (width 0.5) (layer F.Cu) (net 15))
 (segment (start 136.906 99.695) (end 137.16 99.695) (width 0.5) (layer F.Cu) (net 17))
 (segment (start 137.16 99.695) (end 140.335 96.52) (width 0.5) (layer F.Cu) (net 17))
 (segment (start 140.335 96.52) (end 144.145 96.52) (width 0.5) (layer F.Cu) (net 17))
 (segment (start 136.906 86.36) (end 146.812 86.36) (width 0.5) (layer F.Cu) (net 35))
 (segment (start 146.812 86.36) (end 149.352 88.9) (width 0.5) (layer F.Cu) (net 35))
 (segment (start 136.906 95.25) (end 137.16 95.25) (width 0.5) (layer F.Cu) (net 18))
 (segment (start 137.16 95.25) (end 138.43 93.98) (width 0.5) (layer F.Cu) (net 18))
 (segment (start 138.43 93.98) (end 144.145 93.98) (width 0.5) (layer F.Cu) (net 18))
 (segment (start 136.906 97.155) (end 137.16 97.155) (width 0.5) (layer F.Cu) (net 38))
 (segment (start 137.16 97.155) (end 139.065 95.25) (width 0.5) (layer F.Cu) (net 38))
 (segment (start 139.065 95.25) (end 147.955 95.25) (width 0.5) (layer F.Cu) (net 38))
 (segment (start 147.955 95.25) (end 149.225 93.98) (width 0.5) (layer F.Cu) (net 38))
 (segment (start 136.906 90.805) (end 137.541 90.17) (width 0.5) (layer F.Cu) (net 36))
 (segment (start 137.541 90.17) (end 147.955 90.17) (width 0.5) (layer F.Cu) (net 36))
 (segment (start 147.955 90.17) (end 149.225 91.44) (width 0.5) (layer F.Cu) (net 36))
 (segment (start 136.906 101.6) (end 137.16 101.6) (width 0.5) (layer F.Cu) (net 37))
 (segment (start 140.850001 97.909999) (end 147.835001 97.909999) (width 0.5) (layer F.Cu) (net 37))
 (segment (start 137.16 101.6) (end 140.850001 97.909999) (width 0.5) (layer F.Cu) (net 37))
 (segment (start 147.835001 97.909999) (end 149.225 96.52) (width 0.5) (layer F.Cu) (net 37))
 (segment (start 159.766 88.9) (end 169.545 88.9) (width 0.5) (layer F.Cu) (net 31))
 (segment (start 157.226 88.9) (end 159.766 88.9) (width 0.5) (layer F.Cu) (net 31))
 (segment (start 157.226 92.71) (end 157.48 92.71) (width 0.5) (layer F.Cu) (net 32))
 (segment (start 160.02 92.71) (end 161.29 91.44) (width 0.5) (layer F.Cu) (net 32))
 (segment (start 161.29 91.44) (end 168.91 91.44) (width 0.5) (layer F.Cu) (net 32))
 (segment (start 160.02 92.71) (end 157.48 92.71) (width 0.5) (layer F.Cu) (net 32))
 (segment (start 157.226 95.25) (end 157.48 95.25) (width 0.5) (layer F.Cu) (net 34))
 (segment (start 160.02 95.25) (end 161.29 93.98) (width 0.5) (layer F.Cu) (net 34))
 (segment (start 161.29 93.98) (end 168.91 93.98) (width 0.5) (layer F.Cu) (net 34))
 (segment (start 157.226 95.25) (end 160.02 95.25) (width 0.5) (layer F.Cu) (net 34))
 (segment (start 157.226 99.06) (end 157.48 99.06) (width 0.5) (layer F.Cu) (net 33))
 (segment (start 160.02 99.06) (end 162.56 96.52) (width 0.5) (layer F.Cu) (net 33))
 (segment (start 162.56 96.52) (end 169.545 96.52) (width 0.5) (layer F.Cu) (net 33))
 (segment (start 160.02 99.06) (end 157.48 99.06) (width 0.5) (layer F.Cu) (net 33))
 (segment (start 159.766 86.995) (end 172.085 86.995) (width 0.5) (layer F.Cu) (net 27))
 (segment (start 172.32 86.995) (end 172.085 86.995) (width 0.5) (layer F.Cu) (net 27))
 (segment (start 174.225 88.9) (end 172.32 86.995) (width 0.5) (layer F.Cu) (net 27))
 (segment (start 159.766 86.995) (end 157.48 86.995) (width 0.5) (layer F.Cu) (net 27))
 (segment (start 157.226 97.155) (end 157.48 97.155) (width 0.5) (layer F.Cu) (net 30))
 (segment (start 160.02 97.155) (end 161.925 95.25) (width 0.5) (layer F.Cu) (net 30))
 (segment (start 161.925 95.25) (end 172.72 95.25) (width 0.5) (layer F.Cu) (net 30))
 (segment (start 172.72 95.25) (end 173.99 93.98) (width 0.5) (layer F.Cu) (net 30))
 (segment (start 157.226 97.155) (end 160.02 97.155) (width 0.5) (layer F.Cu) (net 30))
 (segment (start 174.225 91.44) (end 173.074999 90.289999) (width 0.5) (layer F.Cu) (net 28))
 (segment (start 161.409999 90.289999) (end 160.535001 90.289999) (width 0.5) (layer F.Cu) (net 28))
 (segment (start 173.074999 90.289999) (end 161.409999 90.289999) (width 0.5) (layer F.Cu) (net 28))
 (segment (start 160.535001 90.289999) (end 160.02 90.805) (width 0.5) (layer F.Cu) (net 28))
 (segment (start 157.226 90.805) (end 160.02 90.805) (width 0.5) (layer F.Cu) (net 28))
 (segment (start 157.226 100.965) (end 157.48 100.965) (width 0.5) (layer F.Cu) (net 29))
 (segment (start 160.02 100.965) (end 163.195 97.79) (width 0.5) (layer F.Cu) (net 29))
 (segment (start 163.195 97.79) (end 172.72 97.79) (width 0.5) (layer F.Cu) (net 29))
 (segment (start 172.72 97.79) (end 173.99 96.52) (width 0.5) (layer F.Cu) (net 29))
 (segment (start 157.226 100.965) (end 160.02 100.965) (width 0.5) (layer F.Cu) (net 29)))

